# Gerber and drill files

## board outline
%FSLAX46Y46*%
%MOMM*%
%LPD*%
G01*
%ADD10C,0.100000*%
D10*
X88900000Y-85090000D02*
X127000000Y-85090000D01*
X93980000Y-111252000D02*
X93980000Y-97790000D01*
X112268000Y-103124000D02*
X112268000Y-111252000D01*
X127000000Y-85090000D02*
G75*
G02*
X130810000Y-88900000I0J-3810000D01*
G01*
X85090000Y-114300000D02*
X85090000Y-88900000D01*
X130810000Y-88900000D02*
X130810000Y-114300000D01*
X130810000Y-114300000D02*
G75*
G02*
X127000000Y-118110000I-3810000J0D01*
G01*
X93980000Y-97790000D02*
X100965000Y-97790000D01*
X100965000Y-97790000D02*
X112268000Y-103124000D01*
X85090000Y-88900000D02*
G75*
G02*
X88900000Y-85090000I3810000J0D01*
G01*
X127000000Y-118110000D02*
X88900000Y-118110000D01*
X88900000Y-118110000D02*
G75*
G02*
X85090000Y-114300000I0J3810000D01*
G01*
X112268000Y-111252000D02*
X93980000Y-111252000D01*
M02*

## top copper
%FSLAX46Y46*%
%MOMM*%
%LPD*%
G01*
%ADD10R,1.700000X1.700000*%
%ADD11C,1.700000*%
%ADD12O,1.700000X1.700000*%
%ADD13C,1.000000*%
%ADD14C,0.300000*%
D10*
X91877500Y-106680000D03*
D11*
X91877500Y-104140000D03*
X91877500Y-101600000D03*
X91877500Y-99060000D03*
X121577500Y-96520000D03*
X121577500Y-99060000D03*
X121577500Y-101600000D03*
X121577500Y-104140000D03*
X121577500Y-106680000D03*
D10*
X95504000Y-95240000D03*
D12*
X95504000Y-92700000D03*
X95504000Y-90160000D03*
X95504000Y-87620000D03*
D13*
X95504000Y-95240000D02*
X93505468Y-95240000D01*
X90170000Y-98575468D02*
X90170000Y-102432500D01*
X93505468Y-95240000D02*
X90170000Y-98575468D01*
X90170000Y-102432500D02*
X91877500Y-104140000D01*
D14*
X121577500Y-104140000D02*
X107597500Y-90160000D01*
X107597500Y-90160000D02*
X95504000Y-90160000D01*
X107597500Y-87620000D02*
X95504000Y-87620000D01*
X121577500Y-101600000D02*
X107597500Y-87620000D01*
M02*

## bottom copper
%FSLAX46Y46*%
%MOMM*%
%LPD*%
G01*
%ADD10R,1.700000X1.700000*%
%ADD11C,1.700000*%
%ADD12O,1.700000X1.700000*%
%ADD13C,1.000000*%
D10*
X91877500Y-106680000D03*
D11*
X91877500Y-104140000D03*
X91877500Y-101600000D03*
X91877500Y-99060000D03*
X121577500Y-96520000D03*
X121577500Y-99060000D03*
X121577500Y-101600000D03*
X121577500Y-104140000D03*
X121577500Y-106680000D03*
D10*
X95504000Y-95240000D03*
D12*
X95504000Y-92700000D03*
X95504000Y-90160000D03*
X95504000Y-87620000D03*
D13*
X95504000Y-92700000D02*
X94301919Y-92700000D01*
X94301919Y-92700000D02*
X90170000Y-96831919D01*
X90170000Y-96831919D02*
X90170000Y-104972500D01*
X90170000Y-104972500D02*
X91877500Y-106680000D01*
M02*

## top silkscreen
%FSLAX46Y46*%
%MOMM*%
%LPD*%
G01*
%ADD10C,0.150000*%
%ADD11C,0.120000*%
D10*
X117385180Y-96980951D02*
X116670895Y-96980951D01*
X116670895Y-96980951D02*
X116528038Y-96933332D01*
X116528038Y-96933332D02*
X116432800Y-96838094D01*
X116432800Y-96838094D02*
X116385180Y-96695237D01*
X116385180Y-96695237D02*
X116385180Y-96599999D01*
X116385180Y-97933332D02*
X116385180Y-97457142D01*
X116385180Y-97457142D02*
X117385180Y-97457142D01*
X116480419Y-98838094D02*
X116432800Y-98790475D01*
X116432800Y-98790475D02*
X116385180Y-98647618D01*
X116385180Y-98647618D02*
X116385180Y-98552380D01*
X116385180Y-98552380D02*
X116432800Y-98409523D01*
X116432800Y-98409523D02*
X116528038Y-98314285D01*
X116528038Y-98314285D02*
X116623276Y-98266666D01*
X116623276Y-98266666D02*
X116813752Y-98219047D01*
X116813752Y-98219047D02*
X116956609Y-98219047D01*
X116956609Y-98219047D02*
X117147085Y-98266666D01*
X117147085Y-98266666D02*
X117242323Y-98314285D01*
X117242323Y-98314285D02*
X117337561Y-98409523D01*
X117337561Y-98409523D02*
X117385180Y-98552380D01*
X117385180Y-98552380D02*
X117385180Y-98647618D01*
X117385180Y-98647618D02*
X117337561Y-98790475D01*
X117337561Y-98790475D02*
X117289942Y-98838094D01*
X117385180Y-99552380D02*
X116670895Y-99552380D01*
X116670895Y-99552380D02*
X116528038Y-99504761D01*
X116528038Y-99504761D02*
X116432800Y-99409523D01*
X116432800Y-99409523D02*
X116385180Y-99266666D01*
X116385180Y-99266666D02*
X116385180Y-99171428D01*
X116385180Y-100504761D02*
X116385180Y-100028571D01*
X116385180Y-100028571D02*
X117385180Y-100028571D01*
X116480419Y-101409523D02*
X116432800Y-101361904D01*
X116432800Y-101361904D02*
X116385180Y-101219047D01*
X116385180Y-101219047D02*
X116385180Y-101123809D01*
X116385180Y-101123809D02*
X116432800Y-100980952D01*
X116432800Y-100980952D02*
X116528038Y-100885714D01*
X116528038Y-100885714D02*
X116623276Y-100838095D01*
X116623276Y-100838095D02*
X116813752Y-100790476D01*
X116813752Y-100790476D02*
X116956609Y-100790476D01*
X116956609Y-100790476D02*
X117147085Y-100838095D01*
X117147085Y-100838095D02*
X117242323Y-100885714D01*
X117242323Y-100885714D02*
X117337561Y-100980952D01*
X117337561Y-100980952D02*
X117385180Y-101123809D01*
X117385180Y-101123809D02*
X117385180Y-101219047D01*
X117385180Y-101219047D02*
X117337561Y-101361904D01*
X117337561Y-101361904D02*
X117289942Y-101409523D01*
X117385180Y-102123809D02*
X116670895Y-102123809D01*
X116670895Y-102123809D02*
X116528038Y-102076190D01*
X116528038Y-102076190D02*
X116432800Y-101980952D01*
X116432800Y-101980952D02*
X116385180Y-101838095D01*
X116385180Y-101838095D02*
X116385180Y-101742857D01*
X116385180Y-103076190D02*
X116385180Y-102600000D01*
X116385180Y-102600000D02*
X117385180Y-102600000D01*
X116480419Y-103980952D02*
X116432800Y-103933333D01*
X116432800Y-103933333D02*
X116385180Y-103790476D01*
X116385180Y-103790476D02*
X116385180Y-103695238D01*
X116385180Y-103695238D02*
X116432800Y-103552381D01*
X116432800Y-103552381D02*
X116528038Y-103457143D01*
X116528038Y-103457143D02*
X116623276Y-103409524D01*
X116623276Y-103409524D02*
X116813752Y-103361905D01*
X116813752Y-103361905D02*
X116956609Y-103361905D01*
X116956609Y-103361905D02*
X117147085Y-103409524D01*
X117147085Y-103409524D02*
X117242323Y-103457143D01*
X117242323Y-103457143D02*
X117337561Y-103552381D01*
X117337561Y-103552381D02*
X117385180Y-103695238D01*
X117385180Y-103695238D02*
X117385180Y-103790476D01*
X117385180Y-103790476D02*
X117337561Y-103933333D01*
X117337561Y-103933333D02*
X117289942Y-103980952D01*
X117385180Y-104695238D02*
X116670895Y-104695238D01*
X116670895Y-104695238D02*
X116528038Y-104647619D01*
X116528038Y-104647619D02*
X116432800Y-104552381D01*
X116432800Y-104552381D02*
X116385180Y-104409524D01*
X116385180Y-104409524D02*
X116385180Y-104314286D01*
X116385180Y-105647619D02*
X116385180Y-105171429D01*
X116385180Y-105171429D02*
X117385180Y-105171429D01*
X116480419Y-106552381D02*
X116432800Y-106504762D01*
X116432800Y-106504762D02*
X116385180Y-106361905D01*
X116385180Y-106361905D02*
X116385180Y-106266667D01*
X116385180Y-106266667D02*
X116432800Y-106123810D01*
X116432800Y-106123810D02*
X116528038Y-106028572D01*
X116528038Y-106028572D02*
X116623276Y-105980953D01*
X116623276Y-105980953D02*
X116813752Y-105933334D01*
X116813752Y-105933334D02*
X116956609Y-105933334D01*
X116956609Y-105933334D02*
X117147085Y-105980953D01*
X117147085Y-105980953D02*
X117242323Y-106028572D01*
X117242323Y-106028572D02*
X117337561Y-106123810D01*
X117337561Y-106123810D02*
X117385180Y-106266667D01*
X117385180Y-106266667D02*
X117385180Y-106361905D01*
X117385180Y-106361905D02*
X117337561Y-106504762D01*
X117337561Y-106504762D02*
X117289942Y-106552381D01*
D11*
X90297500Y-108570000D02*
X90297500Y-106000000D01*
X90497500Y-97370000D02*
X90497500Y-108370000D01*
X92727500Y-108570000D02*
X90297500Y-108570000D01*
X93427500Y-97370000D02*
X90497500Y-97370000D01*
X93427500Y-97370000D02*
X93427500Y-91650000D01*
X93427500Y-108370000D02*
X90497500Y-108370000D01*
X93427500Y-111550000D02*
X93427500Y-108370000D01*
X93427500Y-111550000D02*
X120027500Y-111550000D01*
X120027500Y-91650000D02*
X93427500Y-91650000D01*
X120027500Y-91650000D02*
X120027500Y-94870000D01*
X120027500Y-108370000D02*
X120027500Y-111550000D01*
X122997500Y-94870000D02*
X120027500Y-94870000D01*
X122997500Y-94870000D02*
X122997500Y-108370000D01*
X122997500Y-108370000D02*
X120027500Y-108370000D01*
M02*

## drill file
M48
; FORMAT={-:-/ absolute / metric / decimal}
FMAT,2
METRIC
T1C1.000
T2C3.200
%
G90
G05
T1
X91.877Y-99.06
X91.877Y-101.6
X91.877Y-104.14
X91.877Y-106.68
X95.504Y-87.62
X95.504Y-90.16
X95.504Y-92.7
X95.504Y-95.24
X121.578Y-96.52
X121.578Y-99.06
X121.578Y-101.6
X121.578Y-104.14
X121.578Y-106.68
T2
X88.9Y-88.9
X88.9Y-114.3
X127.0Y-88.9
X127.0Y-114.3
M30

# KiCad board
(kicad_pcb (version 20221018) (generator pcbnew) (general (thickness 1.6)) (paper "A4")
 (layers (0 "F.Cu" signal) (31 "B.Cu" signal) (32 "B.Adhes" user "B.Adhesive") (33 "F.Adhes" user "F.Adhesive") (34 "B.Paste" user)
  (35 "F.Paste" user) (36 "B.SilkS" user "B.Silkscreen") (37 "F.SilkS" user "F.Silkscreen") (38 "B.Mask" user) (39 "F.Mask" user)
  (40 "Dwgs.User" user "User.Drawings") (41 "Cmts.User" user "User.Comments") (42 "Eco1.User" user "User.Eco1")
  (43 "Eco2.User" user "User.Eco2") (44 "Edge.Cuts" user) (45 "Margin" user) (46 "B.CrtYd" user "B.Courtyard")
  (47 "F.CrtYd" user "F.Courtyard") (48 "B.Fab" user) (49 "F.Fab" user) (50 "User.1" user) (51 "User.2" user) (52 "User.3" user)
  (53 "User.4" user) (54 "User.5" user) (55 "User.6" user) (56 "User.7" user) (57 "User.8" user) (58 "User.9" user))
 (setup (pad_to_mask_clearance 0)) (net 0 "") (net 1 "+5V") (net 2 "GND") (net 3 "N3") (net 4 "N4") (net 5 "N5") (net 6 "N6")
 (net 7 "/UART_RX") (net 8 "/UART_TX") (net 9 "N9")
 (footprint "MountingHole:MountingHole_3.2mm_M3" (layer "F.Cu") (at 88.9 114.3)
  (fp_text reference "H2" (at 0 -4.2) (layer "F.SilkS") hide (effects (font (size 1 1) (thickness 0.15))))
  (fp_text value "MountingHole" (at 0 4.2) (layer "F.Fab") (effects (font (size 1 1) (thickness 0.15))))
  (pad "" np_thru_hole circle (at 0 0) (size 3.2 3.2) (drill 3.2) (layers "*.Cu" "*.Mask")))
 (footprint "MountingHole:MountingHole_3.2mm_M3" (layer "F.Cu") (at 127 88.9)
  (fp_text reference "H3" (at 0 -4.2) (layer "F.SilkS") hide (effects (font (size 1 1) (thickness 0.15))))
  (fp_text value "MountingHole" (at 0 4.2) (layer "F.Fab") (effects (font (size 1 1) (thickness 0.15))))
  (pad "" np_thru_hole circle (at 0 0) (size 3.2 3.2) (drill 3.2) (layers "*.Cu" "*.Mask")))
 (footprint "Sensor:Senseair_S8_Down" (layer "F.Cu") (at 91.8775 106.68)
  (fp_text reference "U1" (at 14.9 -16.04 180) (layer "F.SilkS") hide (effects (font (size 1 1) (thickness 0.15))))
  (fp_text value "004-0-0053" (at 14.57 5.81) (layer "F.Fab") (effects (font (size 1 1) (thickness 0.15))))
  (fp_line (start -1.58 1.89) (end -1.58 -0.68) (stroke (width 0.12) (type solid)) (layer "F.SilkS"))
  (fp_line (start -1.38 -9.31) (end -1.38 1.69) (stroke (width 0.12) (type solid)) (layer "F.SilkS"))
  (fp_line (start 0.85 1.89) (end -1.58 1.89) (stroke (width 0.12) (type solid)) (layer "F.SilkS"))
  (fp_line (start 1.55 -9.31) (end -1.38 -9.31) (stroke (width 0.12) (type solid)) (layer "F.SilkS"))
  (fp_line (start 1.55 -9.31) (end 1.55 -15.03) (stroke (width 0.12) (type solid)) (layer "F.SilkS"))
  (fp_line (start 1.55 1.69) (end -1.38 1.69) (stroke (width 0.12) (type solid)) (layer "F.SilkS"))
  (fp_line (start 1.55 4.87) (end 1.55 1.69) (stroke (width 0.12) (type solid)) (layer "F.SilkS"))
  (fp_line (start 1.55 4.87) (end 28.15 4.87) (stroke (width 0.12) (type solid)) (layer "F.SilkS"))
  (fp_line (start 28.15 -15.03) (end 1.55 -15.03) (stroke (width 0.12) (type solid)) (layer "F.SilkS"))
  (fp_line (start 28.15 -15.03) (end 28.15 -11.81) (stroke (width 0.12) (type solid)) (layer "F.SilkS"))
  (fp_line (start 28.15 1.69) (end 28.15 4.87) (stroke (width 0.12) (type solid)) (layer "F.SilkS"))
  (fp_line (start 31.12 -11.81) (end 28.15 -11.81) (stroke (width 0.12) (type solid)) (layer "F.SilkS"))
  (fp_line (start 31.12 -11.81) (end 31.12 1.69) (stroke (width 0.12) (type solid)) (layer "F.SilkS"))
  (fp_line (start 31.12 1.69) (end 28.15 1.69) (stroke (width 0.12) (type solid)) (layer "F.SilkS"))
  (pad "1" thru_hole rect (at 0 0) (size 1.7 1.7) (drill 1) (layers "*.Cu" "*.Mask") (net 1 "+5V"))
  (pad "2" thru_hole circle (at 0 -2.54) (size 1.7 1.7) (drill 1) (layers "*.Cu" "*.Mask") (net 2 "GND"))
  (pad "3" thru_hole circle (at 0 -5.08) (size 1.7 1.7) (drill 1) (layers "*.Cu" "*.Mask") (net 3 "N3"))
  (pad "4" thru_hole circle (at 0 -7.62) (size 1.7 1.7) (drill 1) (layers "*.Cu" "*.Mask") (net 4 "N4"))
  (pad "5" thru_hole circle (at 29.7 -10.16) (size 1.7 1.7) (drill 1) (layers "*.Cu" "*.Mask") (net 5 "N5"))
  (pad "6" thru_hole circle (at 29.7 -7.62) (size 1.7 1.7) (drill 1) (layers "*.Cu" "*.Mask") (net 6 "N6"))
  (pad "7" thru_hole circle (at 29.7 -5.08) (size 1.7 1.7) (drill 1) (layers "*.Cu" "*.Mask") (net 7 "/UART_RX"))
  (pad "8" thru_hole circle (at 29.7 -2.54) (size 1.7 1.7) (drill 1) (layers "*.Cu" "*.Mask") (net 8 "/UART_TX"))
  (pad "9" thru_hole circle (at 29.7 0) (size 1.7 1.7) (drill 1) (layers "*.Cu" "*.Mask") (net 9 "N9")))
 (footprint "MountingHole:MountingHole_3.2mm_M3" (layer "F.Cu") (at 88.9 88.9)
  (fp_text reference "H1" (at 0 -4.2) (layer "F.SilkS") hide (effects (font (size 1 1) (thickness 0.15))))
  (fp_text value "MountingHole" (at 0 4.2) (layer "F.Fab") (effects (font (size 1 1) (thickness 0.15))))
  (pad "" np_thru_hole circle (at 0 0) (size 3.2 3.2) (drill 3.2) (layers "*.Cu" "*.Mask")))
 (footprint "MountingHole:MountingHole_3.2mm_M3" (layer "F.Cu") (at 127 114.3)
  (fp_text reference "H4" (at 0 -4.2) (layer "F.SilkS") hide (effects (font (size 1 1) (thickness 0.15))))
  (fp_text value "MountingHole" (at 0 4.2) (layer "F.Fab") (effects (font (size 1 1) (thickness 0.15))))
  (pad "" np_thru_hole circle (at 0 0) (size 3.2 3.2) (drill 3.2) (layers "*.Cu" "*.Mask")))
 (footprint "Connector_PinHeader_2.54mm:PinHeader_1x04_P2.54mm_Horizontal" (layer "B.Cu") (at 95.504 95.24)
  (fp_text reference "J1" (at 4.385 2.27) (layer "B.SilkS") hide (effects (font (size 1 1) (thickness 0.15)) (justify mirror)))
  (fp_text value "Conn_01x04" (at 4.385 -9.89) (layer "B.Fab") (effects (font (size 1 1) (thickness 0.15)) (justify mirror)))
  (pad "1" thru_hole rect (at 0 0) (size 1.7 1.7) (drill 1) (layers "*.Cu" "*.Mask") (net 2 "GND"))
  (pad "2" thru_hole oval (at 0 -2.54) (size 1.7 1.7) (drill 1) (layers "*.Cu" "*.Mask") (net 1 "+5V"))
  (pad "3" thru_hole oval (at 0 -5.08) (size 1.7 1.7) (drill 1) (layers "*.Cu" "*.Mask") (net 8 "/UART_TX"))
  (pad "4" thru_hole oval (at 0 -7.62) (size 1.7 1.7) (drill 1) (layers "*.Cu" "*.Mask") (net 7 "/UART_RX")))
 (gr_line (start 88.9 85.09) (end 127 85.09) (stroke (width 0.1) (type default)) (layer "Edge.Cuts"))
 (gr_line (start 93.98 111.252) (end 93.98 97.79) (stroke (width 0.1) (type default)) (layer "Edge.Cuts"))
 (gr_line (start 112.268 103.124) (end 112.268 111.252) (stroke (width 0.1) (type default)) (layer "Edge.Cuts"))
 (gr_arc (start 127 85.09) (mid 129.694077 86.205923) (end 130.81 88.9) (stroke (width 0.1) (type default)) (layer "Edge.Cuts"))
 (gr_line (start 85.09 114.3) (end 85.09 88.9) (stroke (width 0.1) (type default)) (layer "Edge.Cuts"))
 (gr_line (start 130.81 88.9) (end 130.81 114.3) (stroke (width 0.1) (type default)) (layer "Edge.Cuts"))
 (gr_arc (start 130.81 114.3) (mid 129.694077 116.994077) (end 127 118.11) (stroke (width 0.1) (type default)) (layer "Edge.Cuts"))
 (gr_line (start 93.98 97.79) (end 100.965 97.79) (stroke (width 0.1) (type default)) (layer "Edge.Cuts"))
 (gr_line (start 100.965 97.79) (end 112.268 103.124) (stroke (width 0.1) (type default)) (layer "Edge.Cuts"))
 (gr_arc (start 85.09 88.9) (mid 86.205923 86.205923) (end 88.9 85.09) (stroke (width 0.1) (type default)) (layer "Edge.Cuts"))
 (gr_line (start 127 118.11) (end 88.9 118.11) (stroke (width 0.1) (type default)) (layer "Edge.Cuts"))
 (gr_arc (start 88.9 118.11) (mid 86.205923 116.994077) (end 85.09 114.3) (stroke (width 0.1) (type default)) (layer "Edge.Cuts"))
 (gr_line (start 112.268 111.252) (end 93.98 111.252) (stroke (width 0.1) (type default)) (layer "Edge.Cuts"))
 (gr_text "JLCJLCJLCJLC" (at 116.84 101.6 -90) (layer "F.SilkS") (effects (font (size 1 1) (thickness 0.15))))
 (segment (start 95.504 95.24) (end 93.505468 95.24) (width 1) (layer "F.Cu") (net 2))
 (segment (start 90.17 98.575468) (end 90.17 102.4325) (width 1) (layer "F.Cu") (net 2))
 (segment (start 93.505468 95.24) (end 90.17 98.575468) (width 1) (layer "F.Cu") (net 2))
 (segment (start 90.17 102.4325) (end 91.8775 104.14) (width 1) (layer "F.Cu") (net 2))
 (segment (start 95.504 92.7) (end 94.301919 92.7) (width 1) (layer "B.Cu") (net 1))
 (segment (start 94.301919 92.7) (end 90.17 96.831919) (width 1) (layer "B.Cu") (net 1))
 (segment (start 90.17 96.831919) (end 90.17 104.9725) (width 1) (layer "B.Cu") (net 1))
 (segment (start 90.17 104.9725) (end 91.8775 106.68) (width 1) (layer "B.Cu") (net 1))
 (segment (start 121.5775 104.14) (end 107.5975 90.16) (width 0.3) (layer "F.Cu") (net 8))
 (segment (start 107.5975 90.16) (end 95.504 90.16) (width 0.3) (layer "F.Cu") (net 8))
 (segment (start 107.5975 87.62) (end 95.504 87.62) (width 0.3) (layer "F.Cu") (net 7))
 (segment (start 121.5775 101.6) (end 107.5975 87.62) (width 0.3) (layer "F.Cu") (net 7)))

